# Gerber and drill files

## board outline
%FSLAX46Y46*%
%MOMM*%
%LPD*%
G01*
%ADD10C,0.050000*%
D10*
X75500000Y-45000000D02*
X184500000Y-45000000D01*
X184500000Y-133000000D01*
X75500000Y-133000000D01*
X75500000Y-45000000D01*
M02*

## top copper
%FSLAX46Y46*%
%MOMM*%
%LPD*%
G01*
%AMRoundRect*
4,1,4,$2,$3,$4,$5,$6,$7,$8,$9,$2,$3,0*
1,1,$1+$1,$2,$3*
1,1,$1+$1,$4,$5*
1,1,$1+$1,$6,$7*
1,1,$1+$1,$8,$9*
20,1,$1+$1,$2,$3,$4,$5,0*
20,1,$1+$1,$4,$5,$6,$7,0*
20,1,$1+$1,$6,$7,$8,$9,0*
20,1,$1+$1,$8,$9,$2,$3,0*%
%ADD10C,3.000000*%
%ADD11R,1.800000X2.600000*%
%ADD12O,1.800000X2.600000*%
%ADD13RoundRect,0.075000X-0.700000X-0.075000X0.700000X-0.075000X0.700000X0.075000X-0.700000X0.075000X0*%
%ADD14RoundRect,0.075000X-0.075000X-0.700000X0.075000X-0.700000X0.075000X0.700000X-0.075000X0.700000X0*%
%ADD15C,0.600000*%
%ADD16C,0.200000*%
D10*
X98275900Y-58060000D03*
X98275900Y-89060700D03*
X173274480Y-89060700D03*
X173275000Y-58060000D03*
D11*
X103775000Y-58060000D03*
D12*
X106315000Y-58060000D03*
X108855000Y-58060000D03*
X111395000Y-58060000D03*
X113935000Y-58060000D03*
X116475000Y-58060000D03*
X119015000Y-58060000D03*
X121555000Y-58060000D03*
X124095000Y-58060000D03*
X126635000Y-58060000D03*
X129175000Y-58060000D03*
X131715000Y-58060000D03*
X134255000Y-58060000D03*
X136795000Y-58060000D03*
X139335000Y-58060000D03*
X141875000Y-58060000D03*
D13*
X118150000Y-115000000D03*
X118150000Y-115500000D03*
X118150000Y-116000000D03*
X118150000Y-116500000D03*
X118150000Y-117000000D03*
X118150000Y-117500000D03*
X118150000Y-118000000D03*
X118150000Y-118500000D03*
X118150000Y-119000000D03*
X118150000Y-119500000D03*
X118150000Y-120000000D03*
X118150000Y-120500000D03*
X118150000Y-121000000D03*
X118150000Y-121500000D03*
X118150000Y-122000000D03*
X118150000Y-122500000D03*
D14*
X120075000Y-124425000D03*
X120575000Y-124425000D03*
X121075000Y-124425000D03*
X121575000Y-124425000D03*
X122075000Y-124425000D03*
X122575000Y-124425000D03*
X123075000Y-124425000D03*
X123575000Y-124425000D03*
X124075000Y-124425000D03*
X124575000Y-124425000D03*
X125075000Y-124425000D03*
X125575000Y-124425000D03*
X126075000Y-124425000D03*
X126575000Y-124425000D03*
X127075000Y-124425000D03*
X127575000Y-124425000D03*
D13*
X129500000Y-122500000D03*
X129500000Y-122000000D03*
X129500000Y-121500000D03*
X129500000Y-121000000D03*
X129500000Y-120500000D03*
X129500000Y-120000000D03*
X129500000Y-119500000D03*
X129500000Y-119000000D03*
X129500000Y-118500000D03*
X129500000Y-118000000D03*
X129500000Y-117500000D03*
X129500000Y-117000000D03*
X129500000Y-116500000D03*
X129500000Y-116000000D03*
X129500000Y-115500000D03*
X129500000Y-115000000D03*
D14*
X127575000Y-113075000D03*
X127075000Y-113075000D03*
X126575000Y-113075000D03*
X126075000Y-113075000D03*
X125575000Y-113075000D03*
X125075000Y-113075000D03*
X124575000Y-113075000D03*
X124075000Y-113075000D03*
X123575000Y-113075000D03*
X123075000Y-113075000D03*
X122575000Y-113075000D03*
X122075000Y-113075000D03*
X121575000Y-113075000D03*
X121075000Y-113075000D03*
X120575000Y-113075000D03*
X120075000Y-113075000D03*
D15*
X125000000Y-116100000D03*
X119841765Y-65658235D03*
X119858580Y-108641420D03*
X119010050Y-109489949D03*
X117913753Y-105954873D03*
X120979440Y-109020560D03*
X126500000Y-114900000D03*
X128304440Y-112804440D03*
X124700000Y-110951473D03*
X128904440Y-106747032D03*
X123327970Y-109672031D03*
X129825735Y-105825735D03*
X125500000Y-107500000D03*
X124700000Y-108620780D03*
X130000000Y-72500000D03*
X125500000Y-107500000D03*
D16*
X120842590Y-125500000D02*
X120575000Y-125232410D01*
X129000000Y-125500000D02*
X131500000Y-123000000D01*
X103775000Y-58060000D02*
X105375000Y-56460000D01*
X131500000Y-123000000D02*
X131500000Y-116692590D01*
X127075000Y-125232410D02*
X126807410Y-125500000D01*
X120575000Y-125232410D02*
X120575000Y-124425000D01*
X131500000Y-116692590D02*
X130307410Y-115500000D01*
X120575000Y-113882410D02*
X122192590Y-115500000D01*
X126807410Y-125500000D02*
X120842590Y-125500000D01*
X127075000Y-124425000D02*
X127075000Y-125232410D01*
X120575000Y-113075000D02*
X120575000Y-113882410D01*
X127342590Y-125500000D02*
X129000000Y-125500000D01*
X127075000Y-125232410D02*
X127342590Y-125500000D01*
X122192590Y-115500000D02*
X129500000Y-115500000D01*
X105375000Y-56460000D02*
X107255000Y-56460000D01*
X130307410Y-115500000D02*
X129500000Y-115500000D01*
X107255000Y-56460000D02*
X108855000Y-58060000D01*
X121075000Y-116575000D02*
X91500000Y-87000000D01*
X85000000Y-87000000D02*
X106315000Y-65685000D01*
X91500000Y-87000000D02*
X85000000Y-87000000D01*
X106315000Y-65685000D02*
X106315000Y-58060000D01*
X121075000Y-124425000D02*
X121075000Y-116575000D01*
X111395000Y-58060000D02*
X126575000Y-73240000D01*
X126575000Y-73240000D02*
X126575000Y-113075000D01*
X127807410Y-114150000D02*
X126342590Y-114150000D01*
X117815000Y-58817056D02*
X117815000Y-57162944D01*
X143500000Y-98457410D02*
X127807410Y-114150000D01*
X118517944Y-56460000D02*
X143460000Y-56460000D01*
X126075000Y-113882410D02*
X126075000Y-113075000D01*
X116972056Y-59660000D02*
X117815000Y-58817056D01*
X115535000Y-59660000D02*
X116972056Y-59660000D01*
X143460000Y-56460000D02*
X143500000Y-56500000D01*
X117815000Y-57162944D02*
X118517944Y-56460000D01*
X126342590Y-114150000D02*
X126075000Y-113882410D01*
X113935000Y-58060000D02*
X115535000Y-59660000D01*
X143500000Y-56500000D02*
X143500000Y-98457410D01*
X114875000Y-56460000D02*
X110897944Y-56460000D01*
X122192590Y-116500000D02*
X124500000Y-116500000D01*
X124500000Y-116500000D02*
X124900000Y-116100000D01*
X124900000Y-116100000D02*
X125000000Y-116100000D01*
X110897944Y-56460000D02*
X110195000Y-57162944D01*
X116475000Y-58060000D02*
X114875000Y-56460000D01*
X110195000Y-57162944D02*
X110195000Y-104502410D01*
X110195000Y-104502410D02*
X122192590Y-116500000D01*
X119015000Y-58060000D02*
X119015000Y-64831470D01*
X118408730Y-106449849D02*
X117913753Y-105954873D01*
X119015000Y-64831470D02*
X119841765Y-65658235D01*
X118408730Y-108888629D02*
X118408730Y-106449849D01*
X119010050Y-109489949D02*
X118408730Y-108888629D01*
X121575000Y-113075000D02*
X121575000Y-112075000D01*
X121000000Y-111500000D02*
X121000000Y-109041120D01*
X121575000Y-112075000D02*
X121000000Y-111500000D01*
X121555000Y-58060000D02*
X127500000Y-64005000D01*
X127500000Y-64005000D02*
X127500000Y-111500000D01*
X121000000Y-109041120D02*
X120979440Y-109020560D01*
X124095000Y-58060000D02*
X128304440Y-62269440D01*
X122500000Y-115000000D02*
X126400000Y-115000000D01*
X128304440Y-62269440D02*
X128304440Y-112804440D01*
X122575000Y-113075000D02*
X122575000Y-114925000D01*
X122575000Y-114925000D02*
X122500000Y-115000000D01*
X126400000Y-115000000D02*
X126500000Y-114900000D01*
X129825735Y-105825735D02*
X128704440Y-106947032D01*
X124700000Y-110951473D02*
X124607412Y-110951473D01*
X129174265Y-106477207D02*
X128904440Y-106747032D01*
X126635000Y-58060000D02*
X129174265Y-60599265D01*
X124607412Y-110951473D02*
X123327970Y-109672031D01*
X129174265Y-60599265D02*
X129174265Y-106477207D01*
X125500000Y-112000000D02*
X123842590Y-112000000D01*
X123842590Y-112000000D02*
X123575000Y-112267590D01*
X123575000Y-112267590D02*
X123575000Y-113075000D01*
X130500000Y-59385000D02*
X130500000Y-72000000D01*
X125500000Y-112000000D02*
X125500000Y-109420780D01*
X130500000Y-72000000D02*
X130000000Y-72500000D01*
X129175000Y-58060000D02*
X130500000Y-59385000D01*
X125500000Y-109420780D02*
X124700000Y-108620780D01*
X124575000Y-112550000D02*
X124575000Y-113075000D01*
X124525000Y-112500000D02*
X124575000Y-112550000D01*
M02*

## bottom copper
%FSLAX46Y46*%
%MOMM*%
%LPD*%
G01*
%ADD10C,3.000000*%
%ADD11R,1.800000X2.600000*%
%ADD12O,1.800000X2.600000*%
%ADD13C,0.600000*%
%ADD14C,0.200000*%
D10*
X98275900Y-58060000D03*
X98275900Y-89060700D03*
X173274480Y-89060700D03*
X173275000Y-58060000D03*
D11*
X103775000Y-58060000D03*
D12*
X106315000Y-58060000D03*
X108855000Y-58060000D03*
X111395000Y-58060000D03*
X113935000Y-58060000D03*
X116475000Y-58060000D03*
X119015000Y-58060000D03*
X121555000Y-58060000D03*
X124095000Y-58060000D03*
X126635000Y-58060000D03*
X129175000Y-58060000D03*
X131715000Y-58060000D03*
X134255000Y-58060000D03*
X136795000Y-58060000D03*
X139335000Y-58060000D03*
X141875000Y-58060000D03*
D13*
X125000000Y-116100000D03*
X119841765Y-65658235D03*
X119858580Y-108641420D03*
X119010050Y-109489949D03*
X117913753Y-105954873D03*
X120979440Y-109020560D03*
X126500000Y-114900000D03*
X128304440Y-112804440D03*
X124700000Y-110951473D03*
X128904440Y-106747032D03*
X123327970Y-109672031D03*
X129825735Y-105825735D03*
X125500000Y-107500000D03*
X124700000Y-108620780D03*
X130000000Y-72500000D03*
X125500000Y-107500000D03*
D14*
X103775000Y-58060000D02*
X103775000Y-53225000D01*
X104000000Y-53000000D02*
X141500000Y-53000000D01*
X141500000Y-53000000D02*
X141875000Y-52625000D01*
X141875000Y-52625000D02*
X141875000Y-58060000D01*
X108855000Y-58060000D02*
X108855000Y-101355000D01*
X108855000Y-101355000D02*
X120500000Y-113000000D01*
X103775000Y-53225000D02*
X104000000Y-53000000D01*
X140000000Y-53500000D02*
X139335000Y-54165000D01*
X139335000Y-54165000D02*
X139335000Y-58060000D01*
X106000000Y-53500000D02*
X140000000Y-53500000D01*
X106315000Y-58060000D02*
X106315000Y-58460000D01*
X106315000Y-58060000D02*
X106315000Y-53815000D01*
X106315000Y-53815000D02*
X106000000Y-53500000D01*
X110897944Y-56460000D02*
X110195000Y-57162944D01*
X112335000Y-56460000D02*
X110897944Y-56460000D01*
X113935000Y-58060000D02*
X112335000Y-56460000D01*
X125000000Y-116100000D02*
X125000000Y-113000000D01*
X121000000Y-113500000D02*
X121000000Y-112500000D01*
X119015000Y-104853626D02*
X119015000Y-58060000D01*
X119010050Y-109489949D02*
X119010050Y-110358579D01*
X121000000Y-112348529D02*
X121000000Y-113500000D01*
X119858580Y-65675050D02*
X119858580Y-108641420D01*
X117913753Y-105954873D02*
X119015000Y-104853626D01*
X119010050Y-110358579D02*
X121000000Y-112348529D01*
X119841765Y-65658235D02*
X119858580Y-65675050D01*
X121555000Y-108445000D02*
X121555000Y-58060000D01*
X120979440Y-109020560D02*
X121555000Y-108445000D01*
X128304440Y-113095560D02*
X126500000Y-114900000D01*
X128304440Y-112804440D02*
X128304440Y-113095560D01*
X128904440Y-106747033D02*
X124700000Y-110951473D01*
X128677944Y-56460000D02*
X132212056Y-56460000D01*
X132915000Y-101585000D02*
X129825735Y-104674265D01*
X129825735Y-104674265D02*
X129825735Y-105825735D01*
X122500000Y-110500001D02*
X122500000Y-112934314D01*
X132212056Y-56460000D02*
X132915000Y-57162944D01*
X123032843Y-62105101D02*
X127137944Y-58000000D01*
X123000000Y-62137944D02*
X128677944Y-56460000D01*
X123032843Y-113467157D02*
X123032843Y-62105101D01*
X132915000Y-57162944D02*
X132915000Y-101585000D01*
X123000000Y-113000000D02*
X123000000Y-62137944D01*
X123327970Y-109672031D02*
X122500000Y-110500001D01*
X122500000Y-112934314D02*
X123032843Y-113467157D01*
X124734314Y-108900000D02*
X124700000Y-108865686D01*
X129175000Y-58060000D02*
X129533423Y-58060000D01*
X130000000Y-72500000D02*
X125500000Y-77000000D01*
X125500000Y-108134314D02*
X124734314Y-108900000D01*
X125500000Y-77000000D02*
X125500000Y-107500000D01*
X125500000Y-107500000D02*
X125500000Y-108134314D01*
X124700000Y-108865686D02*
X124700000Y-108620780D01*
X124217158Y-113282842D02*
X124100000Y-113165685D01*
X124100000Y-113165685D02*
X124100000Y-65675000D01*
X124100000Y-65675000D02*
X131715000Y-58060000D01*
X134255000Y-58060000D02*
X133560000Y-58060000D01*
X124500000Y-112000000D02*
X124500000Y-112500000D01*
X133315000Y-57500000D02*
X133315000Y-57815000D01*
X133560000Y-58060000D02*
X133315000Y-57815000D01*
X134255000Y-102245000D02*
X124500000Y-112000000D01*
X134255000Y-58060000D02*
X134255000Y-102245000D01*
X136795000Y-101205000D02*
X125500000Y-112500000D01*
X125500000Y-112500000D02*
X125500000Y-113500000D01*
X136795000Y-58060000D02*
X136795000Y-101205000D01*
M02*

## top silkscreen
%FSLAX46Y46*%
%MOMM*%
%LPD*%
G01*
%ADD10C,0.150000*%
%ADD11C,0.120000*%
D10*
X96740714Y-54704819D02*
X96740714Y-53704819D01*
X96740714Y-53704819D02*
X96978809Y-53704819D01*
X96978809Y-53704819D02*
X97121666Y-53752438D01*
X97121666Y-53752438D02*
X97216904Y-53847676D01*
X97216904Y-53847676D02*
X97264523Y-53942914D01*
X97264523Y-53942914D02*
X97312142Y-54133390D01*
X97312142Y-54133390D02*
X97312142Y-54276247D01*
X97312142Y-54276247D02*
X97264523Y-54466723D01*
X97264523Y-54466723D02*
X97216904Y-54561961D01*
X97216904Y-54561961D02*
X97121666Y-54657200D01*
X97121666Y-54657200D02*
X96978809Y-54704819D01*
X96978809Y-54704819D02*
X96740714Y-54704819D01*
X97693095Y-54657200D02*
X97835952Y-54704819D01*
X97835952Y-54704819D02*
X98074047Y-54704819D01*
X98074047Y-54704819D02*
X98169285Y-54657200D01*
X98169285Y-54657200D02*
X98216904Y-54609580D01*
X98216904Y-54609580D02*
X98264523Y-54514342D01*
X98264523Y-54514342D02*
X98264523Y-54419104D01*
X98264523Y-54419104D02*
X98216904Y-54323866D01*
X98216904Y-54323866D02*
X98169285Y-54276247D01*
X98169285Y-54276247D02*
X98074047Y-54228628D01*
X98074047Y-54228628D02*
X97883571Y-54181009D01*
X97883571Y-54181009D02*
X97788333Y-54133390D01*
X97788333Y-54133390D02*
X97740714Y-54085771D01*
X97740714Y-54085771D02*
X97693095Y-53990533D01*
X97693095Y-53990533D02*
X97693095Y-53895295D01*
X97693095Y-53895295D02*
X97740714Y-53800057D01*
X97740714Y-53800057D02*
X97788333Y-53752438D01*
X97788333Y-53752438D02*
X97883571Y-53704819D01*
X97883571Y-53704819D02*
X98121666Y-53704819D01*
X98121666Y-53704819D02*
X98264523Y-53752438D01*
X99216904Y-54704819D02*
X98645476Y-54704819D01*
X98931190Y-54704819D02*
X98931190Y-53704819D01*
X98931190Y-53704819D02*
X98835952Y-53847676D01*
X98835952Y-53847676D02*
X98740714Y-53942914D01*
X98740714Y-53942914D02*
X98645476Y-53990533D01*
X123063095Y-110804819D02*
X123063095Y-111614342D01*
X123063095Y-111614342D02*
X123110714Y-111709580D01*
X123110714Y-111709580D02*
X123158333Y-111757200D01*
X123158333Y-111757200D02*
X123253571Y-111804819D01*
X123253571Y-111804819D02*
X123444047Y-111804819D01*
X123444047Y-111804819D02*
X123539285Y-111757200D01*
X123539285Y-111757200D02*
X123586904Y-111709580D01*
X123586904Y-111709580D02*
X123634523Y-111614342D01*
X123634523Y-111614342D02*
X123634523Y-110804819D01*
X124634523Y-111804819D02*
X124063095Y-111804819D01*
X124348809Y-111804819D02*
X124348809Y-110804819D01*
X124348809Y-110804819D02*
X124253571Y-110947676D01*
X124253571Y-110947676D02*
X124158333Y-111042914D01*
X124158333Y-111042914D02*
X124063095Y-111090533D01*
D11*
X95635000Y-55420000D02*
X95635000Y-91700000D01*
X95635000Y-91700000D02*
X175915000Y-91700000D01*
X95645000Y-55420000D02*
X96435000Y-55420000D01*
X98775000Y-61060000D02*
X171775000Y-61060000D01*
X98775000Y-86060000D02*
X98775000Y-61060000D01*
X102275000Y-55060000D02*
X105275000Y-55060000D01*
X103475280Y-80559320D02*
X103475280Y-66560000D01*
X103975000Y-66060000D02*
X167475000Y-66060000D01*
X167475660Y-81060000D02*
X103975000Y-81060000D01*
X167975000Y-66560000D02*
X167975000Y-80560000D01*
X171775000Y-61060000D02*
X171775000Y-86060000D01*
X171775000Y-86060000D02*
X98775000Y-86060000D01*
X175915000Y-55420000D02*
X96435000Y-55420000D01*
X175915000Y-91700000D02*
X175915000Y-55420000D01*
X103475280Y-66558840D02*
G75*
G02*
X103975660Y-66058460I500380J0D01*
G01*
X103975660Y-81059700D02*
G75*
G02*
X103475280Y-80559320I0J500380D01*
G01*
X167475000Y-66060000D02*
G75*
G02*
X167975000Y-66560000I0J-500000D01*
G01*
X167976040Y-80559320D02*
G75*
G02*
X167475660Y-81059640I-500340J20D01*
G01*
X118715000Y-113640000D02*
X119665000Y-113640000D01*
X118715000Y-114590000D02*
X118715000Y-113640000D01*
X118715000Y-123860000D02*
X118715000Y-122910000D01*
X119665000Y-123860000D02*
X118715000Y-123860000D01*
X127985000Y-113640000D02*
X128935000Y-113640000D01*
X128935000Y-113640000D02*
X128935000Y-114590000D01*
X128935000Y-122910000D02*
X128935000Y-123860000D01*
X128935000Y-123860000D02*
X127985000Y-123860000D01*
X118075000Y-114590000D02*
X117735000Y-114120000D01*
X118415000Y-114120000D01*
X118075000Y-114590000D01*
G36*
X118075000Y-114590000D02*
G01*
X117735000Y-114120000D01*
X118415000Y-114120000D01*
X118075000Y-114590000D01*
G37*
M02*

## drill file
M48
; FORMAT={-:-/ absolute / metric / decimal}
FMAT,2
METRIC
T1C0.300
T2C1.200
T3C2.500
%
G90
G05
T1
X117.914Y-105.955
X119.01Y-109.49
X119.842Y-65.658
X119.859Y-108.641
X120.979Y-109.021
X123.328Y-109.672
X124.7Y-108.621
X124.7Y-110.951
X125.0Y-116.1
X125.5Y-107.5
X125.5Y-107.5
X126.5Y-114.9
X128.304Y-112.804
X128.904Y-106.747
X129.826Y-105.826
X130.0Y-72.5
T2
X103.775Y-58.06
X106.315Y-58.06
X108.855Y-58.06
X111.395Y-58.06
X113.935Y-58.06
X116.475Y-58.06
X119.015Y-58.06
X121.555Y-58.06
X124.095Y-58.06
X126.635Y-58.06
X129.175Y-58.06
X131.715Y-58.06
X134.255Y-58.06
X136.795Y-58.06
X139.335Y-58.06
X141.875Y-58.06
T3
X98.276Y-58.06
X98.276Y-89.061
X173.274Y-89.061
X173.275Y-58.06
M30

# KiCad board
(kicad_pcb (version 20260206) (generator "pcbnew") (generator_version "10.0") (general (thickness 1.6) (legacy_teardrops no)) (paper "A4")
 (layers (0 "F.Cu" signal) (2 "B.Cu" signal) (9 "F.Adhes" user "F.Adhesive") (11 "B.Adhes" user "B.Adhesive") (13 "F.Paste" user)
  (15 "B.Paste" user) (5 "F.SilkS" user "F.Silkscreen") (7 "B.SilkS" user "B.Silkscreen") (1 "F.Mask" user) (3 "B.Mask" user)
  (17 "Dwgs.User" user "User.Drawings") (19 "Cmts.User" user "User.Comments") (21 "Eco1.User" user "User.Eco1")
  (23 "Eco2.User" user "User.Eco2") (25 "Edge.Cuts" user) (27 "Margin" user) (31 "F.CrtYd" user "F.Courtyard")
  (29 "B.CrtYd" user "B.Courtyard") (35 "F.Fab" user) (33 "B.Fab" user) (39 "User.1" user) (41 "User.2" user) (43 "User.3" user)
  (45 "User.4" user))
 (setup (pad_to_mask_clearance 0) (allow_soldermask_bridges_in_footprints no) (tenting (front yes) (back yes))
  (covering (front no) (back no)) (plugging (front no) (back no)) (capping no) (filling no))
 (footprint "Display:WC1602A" (layer "F.Cu") (at 103.775 58.06)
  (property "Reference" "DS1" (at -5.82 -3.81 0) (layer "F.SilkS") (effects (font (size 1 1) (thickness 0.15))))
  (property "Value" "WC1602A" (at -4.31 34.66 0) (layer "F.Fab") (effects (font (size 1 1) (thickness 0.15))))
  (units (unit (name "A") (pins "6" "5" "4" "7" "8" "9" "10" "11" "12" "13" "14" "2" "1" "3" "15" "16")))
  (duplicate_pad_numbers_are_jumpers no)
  (fp_line (start -8.14 -2.64) (end -8.14 33.64) (stroke (width 0.12) (type solid)) (layer "F.SilkS"))
  (fp_line (start -8.14 33.64) (end 72.14 33.64) (stroke (width 0.12) (type solid)) (layer "F.SilkS"))
  (fp_line (start -8.13 -2.64) (end -7.34 -2.64) (stroke (width 0.12) (type solid)) (layer "F.SilkS"))
  (fp_line (start -5 3) (end 68 3) (stroke (width 0.12) (type solid)) (layer "F.SilkS"))
  (fp_line (start -5 28) (end -5 3) (stroke (width 0.12) (type solid)) (layer "F.SilkS"))
  (fp_line (start -1.5 -3) (end 1.5 -3) (stroke (width 0.12) (type solid)) (layer "F.SilkS"))
  (fp_line (start -0.29972 22.49932) (end -0.29972 8.5) (stroke (width 0.12) (type solid)) (layer "F.SilkS"))
  (fp_line (start 0.2 8) (end 63.7 8) (stroke (width 0.12) (type solid)) (layer "F.SilkS"))
  (fp_line (start 63.70066 23) (end 0.2 23) (stroke (width 0.12) (type solid)) (layer "F.SilkS"))
  (fp_line (start 64.2 8.5) (end 64.2 22.5) (stroke (width 0.12) (type solid)) (layer "F.SilkS"))
  (fp_line (start 68 3) (end 68 28) (stroke (width 0.12) (type solid)) (layer "F.SilkS"))
  (fp_line (start 68 28) (end -5 28) (stroke (width 0.12) (type solid)) (layer "F.SilkS"))
  (fp_line (start 72.14 -2.64) (end -7.34 -2.64) (stroke (width 0.12) (type solid)) (layer "F.SilkS"))
  (fp_line (start 72.14 33.64) (end 72.14 -2.64) (stroke (width 0.12) (type solid)) (layer "F.SilkS"))
  (fp_arc (start -0.29972 8.49884) (mid -0.153162 8.145018) (end 0.20066 7.99846) (stroke (width 0.12) (type solid)) (layer "F.SilkS"))
  (fp_arc (start 0.20066 22.9997) (mid -0.153162 22.853142) (end -0.29972 22.49932) (stroke (width 0.12) (type solid)) (layer "F.SilkS"))
  (fp_arc (start 63.7 8) (mid 64.053553 8.146447) (end 64.2 8.5) (stroke (width 0.12) (type solid)) (layer "F.SilkS"))
  (fp_arc (start 64.20104 22.49932) (mid 64.054482 22.853142) (end 63.70066 22.9997) (stroke (width 0.12) (type solid)) (layer "F.SilkS"))
  (pad "" thru_hole circle (at -5.4991 0) (size 3 3) (drill 2.5) (layers "*.Cu" "*.Mask") (remove_unused_layers no))
  (pad "" thru_hole circle (at -5.4991 31.0007) (size 3 3) (drill 2.5) (layers "*.Cu" "*.Mask") (remove_unused_layers no))
  (pad "" thru_hole circle (at 69.49948 31.0007) (size 3 3) (drill 2.5) (layers "*.Cu" "*.Mask") (remove_unused_layers no))
  (pad "" thru_hole circle (at 69.5 0) (size 3 3) (drill 2.5) (layers "*.Cu" "*.Mask") (remove_unused_layers no))
  (pad "1" thru_hole rect (at 0 0) (size 1.8 2.6) (drill 1.2) (layers "*.Cu" "*.Mask") (remove_unused_layers no) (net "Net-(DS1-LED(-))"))
  (pad "2" thru_hole oval (at 2.54 0) (size 1.8 2.6) (drill 1.2) (layers "*.Cu" "*.Mask") (remove_unused_layers no) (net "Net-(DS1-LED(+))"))
  (pad "3" thru_hole oval (at 5.08 0) (size 1.8 2.6) (drill 1.2) (layers "*.Cu" "*.Mask") (remove_unused_layers no) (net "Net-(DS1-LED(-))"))
  (pad "4" thru_hole oval (at 7.62 0) (size 1.8 2.6) (drill 1.2) (layers "*.Cu" "*.Mask") (remove_unused_layers no) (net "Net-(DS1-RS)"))
  (pad "5" thru_hole oval (at 10.16 0) (size 1.8 2.6) (drill 1.2) (layers "*.Cu" "*.Mask") (remove_unused_layers no)
   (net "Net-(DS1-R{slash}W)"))
  (pad "6" thru_hole oval (at 12.7 0) (size 1.8 2.6) (drill 1.2) (layers "*.Cu" "*.Mask") (remove_unused_layers no) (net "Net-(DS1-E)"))
  (pad "7" thru_hole oval (at 15.24 0) (size 1.8 2.6) (drill 1.2) (layers "*.Cu" "*.Mask") (remove_unused_layers no) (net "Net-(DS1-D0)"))
  (pad "8" thru_hole oval (at 17.78 0) (size 1.8 2.6) (drill 1.2) (layers "*.Cu" "*.Mask") (remove_unused_layers no) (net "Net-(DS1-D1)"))
  (pad "9" thru_hole oval (at 20.32 0) (size 1.8 2.6) (drill 1.2) (layers "*.Cu" "*.Mask") (remove_unused_layers no) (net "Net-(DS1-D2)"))
  (pad "10" thru_hole oval (at 22.86 0) (size 1.8 2.6) (drill 1.2) (layers "*.Cu" "*.Mask") (remove_unused_layers no) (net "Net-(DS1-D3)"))
  (pad "11" thru_hole oval (at 25.4 0) (size 1.8 2.6) (drill 1.2) (layers "*.Cu" "*.Mask") (remove_unused_layers no) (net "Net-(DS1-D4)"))
  (pad "12" thru_hole oval (at 27.94 0) (size 1.8 2.6) (drill 1.2) (layers "*.Cu" "*.Mask") (remove_unused_layers no) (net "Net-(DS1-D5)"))
  (pad "13" thru_hole oval (at 30.48 0) (size 1.8 2.6) (drill 1.2) (layers "*.Cu" "*.Mask") (remove_unused_layers no) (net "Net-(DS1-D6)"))
  (pad "14" thru_hole oval (at 33.02 0) (size 1.8 2.6) (drill 1.2) (layers "*.Cu" "*.Mask") (remove_unused_layers no) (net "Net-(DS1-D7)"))
  (pad "15" thru_hole oval (at 35.56 0) (size 1.8 2.6) (drill 1.2) (layers "*.Cu" "*.Mask") (remove_unused_layers no)
   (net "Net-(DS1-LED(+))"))
  (pad "16" thru_hole oval (at 38.1 0) (size 1.8 2.6) (drill 1.2) (layers "*.Cu" "*.Mask") (remove_unused_layers no)
   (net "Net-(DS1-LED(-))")))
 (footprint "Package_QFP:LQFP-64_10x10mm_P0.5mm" (layer "F.Cu") (at 123.825 118.75)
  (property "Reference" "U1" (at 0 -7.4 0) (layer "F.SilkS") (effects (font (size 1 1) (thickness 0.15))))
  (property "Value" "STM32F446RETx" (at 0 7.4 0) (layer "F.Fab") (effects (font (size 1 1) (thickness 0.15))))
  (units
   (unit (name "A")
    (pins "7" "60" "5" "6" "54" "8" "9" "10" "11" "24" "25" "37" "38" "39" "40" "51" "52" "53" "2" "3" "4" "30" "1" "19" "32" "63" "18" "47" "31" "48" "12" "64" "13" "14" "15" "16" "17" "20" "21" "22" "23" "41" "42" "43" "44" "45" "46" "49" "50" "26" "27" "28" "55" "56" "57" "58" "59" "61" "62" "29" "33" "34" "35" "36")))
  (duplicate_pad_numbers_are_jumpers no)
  (fp_line (start -5.11 -5.11) (end -4.16 -5.11) (stroke (width 0.12) (type solid)) (layer "F.SilkS"))
  (fp_line (start -5.11 -4.16) (end -5.11 -5.11) (stroke (width 0.12) (type solid)) (layer "F.SilkS"))
  (fp_line (start -5.11 5.11) (end -5.11 4.16) (stroke (width 0.12) (type solid)) (layer "F.SilkS"))
  (fp_line (start -4.16 5.11) (end -5.11 5.11) (stroke (width 0.12) (type solid)) (layer "F.SilkS"))
  (fp_line (start 4.16 -5.11) (end 5.11 -5.11) (stroke (width 0.12) (type solid)) (layer "F.SilkS"))
  (fp_line (start 5.11 -5.11) (end 5.11 -4.16) (stroke (width 0.12) (type solid)) (layer "F.SilkS"))
  (fp_line (start 5.11 4.16) (end 5.11 5.11) (stroke (width 0.12) (type solid)) (layer "F.SilkS"))
  (fp_line (start 5.11 5.11) (end 4.16 5.11) (stroke (width 0.12) (type solid)) (layer "F.SilkS"))
  (fp_poly (pts (xy -5.75 -4.16) (xy -6.09 -4.63) (xy -5.41 -4.63)) (stroke (width 0.12) (type solid)) (fill yes) (layer "F.SilkS"))
  (pad "1" smd roundrect (at -5.675 -3.75) (size 1.55 0.3) (layers "F.Cu" "F.Mask" "F.Paste") (roundrect_rratio 0.25)
   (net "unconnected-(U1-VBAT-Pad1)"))
  (pad "2" smd roundrect (at -5.675 -3.25) (size 1.55 0.3) (layers "F.Cu" "F.Mask" "F.Paste") (roundrect_rratio 0.25)
   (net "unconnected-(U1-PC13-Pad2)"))
  (pad "3" smd roundrect (at -5.675 -2.75) (size 1.55 0.3) (layers "F.Cu" "F.Mask" "F.Paste") (roundrect_rratio 0.25)
   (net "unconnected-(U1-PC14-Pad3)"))
  (pad "4" smd roundrect (at -5.675 -2.25) (size 1.55 0.3) (layers "F.Cu" "F.Mask" "F.Paste") (roundrect_rratio 0.25)
   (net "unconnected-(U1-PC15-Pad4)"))
  (pad "5" smd roundrect (at -5.675 -1.75) (size 1.55 0.3) (layers "F.Cu" "F.Mask" "F.Paste") (roundrect_rratio 0.25)
   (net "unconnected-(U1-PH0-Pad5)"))
  (pad "6" smd roundrect (at -5.675 -1.25) (size 1.55 0.3) (layers "F.Cu" "F.Mask" "F.Paste") (roundrect_rratio 0.25)
   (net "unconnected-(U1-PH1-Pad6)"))
  (pad "7" smd roundrect (at -5.675 -0.75) (size 1.55 0.3) (layers "F.Cu" "F.Mask" "F.Paste") (roundrect_rratio 0.25)
   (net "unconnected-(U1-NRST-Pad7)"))
  (pad "8" smd roundrect (at -5.675 -0.25) (size 1.55 0.3) (layers "F.Cu" "F.Mask" "F.Paste") (roundrect_rratio 0.25)
   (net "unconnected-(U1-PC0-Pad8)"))
  (pad "9" smd roundrect (at -5.675 0.25) (size 1.55 0.3) (layers "F.Cu" "F.Mask" "F.Paste") (roundrect_rratio 0.25)
   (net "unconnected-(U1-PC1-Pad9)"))
  (pad "10" smd roundrect (at -5.675 0.75) (size 1.55 0.3) (layers "F.Cu" "F.Mask" "F.Paste") (roundrect_rratio 0.25)
   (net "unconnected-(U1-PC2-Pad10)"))
  (pad "11" smd roundrect (at -5.675 1.25) (size 1.55 0.3) (layers "F.Cu" "F.Mask" "F.Paste") (roundrect_rratio 0.25)
   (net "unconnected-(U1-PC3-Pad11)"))
  (pad "12" smd roundrect (at -5.675 1.75) (size 1.55 0.3) (layers "F.Cu" "F.Mask" "F.Paste") (roundrect_rratio 0.25)
   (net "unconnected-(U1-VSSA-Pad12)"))
  (pad "13" smd roundrect (at -5.675 2.25) (size 1.55 0.3) (layers "F.Cu" "F.Mask" "F.Paste") (roundrect_rratio 0.25)
   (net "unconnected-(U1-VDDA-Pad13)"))
  (pad "14" smd roundrect (at -5.675 2.75) (size 1.55 0.3) (layers "F.Cu" "F.Mask" "F.Paste") (roundrect_rratio 0.25)
   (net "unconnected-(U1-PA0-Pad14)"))
  (pad "15" smd roundrect (at -5.675 3.25) (size 1.55 0.3) (layers "F.Cu" "F.Mask" "F.Paste") (roundrect_rratio 0.25)
   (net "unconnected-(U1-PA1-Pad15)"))
  (pad "16" smd roundrect (at -5.675 3.75) (size 1.55 0.3) (layers "F.Cu" "F.Mask" "F.Paste") (roundrect_rratio 0.25)
   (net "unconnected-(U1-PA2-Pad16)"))
  (pad "17" smd roundrect (at -3.75 5.675) (size 0.3 1.55) (layers "F.Cu" "F.Mask" "F.Paste") (roundrect_rratio 0.25)
   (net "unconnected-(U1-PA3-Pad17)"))
  (pad "18" smd roundrect (at -3.25 5.675) (size 0.3 1.55) (layers "F.Cu" "F.Mask" "F.Paste") (roundrect_rratio 0.25)
   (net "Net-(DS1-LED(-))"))
  (pad "19" smd roundrect (at -2.75 5.675) (size 0.3 1.55) (layers "F.Cu" "F.Mask" "F.Paste") (roundrect_rratio 0.25)
   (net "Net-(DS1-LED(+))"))
  (pad "20" smd roundrect (at -2.25 5.675) (size 0.3 1.55) (layers "F.Cu" "F.Mask" "F.Paste") (roundrect_rratio 0.25)
   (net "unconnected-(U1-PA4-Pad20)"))
  (pad "21" smd roundrect (at -1.75 5.675) (size 0.3 1.55) (layers "F.Cu" "F.Mask" "F.Paste") (roundrect_rratio 0.25)
   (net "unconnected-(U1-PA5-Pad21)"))
  (pad "22" smd roundrect (at -1.25 5.675) (size 0.3 1.55) (layers "F.Cu" "F.Mask" "F.Paste") (roundrect_rratio 0.25)
   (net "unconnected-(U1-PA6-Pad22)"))
  (pad "23" smd roundrect (at -0.75 5.675) (size 0.3 1.55) (layers "F.Cu" "F.Mask" "F.Paste") (roundrect_rratio 0.25)
   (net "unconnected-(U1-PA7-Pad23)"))
  (pad "24" smd roundrect (at -0.25 5.675) (size 0.3 1.55) (layers "F.Cu" "F.Mask" "F.Paste") (roundrect_rratio 0.25)
   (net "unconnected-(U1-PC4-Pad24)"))
  (pad "25" smd roundrect (at 0.25 5.675) (size 0.3 1.55) (layers "F.Cu" "F.Mask" "F.Paste") (roundrect_rratio 0.25)
   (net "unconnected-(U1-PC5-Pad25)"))
  (pad "26" smd roundrect (at 0.75 5.675) (size 0.3 1.55) (layers "F.Cu" "F.Mask" "F.Paste") (roundrect_rratio 0.25)
   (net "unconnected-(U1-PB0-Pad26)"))
  (pad "27" smd roundrect (at 1.25 5.675) (size 0.3 1.55) (layers "F.Cu" "F.Mask" "F.Paste") (roundrect_rratio 0.25)
   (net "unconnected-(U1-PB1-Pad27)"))
  (pad "28" smd roundrect (at 1.75 5.675) (size 0.3 1.55) (layers "F.Cu" "F.Mask" "F.Paste") (roundrect_rratio 0.25)
   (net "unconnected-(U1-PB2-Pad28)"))
  (pad "29" smd roundrect (at 2.25 5.675) (size 0.3 1.55) (layers "F.Cu" "F.Mask" "F.Paste") (roundrect_rratio 0.25)
   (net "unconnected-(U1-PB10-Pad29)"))
  (pad "30" smd roundrect (at 2.75 5.675) (size 0.3 1.55) (layers "F.Cu" "F.Mask" "F.Paste") (roundrect_rratio 0.25)
   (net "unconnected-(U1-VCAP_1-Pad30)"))
  (pad "31" smd roundrect (at 3.25 5.675) (size 0.3 1.55) (layers "F.Cu" "F.Mask" "F.Paste") (roundrect_rratio 0.25)
   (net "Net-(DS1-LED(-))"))
  (pad "32" smd roundrect (at 3.75 5.675) (size 0.3 1.55) (layers "F.Cu" "F.Mask" "F.Paste") (roundrect_rratio 0.25)
   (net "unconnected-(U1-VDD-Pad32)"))
  (pad "33" smd roundrect (at 5.675 3.75) (size 1.55 0.3) (layers "F.Cu" "F.Mask" "F.Paste") (roundrect_rratio 0.25)
   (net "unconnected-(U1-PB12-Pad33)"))
  (pad "34" smd roundrect (at 5.675 3.25) (size 1.55 0.3) (layers "F.Cu" "F.Mask" "F.Paste") (roundrect_rratio 0.25)
   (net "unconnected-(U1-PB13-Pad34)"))
  (pad "35" smd roundrect (at 5.675 2.75) (size 1.55 0.3) (layers "F.Cu" "F.Mask" "F.Paste") (roundrect_rratio 0.25)
   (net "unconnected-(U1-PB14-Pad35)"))
  (pad "36" smd roundrect (at 5.675 2.25) (size 1.55 0.3) (layers "F.Cu" "F.Mask" "F.Paste") (roundrect_rratio 0.25)
   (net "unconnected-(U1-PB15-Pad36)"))
  (pad "37" smd roundrect (at 5.675 1.75) (size 1.55 0.3) (layers "F.Cu" "F.Mask" "F.Paste") (roundrect_rratio 0.25)
   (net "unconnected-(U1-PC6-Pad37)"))
  (pad "38" smd roundrect (at 5.675 1.25) (size 1.55 0.3) (layers "F.Cu" "F.Mask" "F.Paste") (roundrect_rratio 0.25)
   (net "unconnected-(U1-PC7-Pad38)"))
  (pad "39" smd roundrect (at 5.675 0.75) (size 1.55 0.3) (layers "F.Cu" "F.Mask" "F.Paste") (roundrect_rratio 0.25)
   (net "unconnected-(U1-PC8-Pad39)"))
  (pad "40" smd roundrect (at 5.675 0.25) (size 1.55 0.3) (layers "F.Cu" "F.Mask" "F.Paste") (roundrect_rratio 0.25)
   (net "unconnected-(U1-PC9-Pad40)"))
  (pad "41" smd roundrect (at 5.675 -0.25) (size 1.55 0.3) (layers "F.Cu" "F.Mask" "F.Paste") (roundrect_rratio 0.25)
   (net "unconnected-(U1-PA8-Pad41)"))
  (pad "42" smd roundrect (at 5.675 -0.75) (size 1.55 0.3) (layers "F.Cu" "F.Mask" "F.Paste") (roundrect_rratio 0.25)
   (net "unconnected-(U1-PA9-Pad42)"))
  (pad "43" smd roundrect (at 5.675 -1.25) (size 1.55 0.3) (layers "F.Cu" "F.Mask" "F.Paste") (roundrect_rratio 0.25)
   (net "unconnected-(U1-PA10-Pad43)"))
  (pad "44" smd roundrect (at 5.675 -1.75) (size 1.55 0.3) (layers "F.Cu" "F.Mask" "F.Paste") (roundrect_rratio 0.25)
   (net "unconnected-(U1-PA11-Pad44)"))
  (pad "45" smd roundrect (at 5.675 -2.25) (size 1.55 0.3) (layers "F.Cu" "F.Mask" "F.Paste") (roundrect_rratio 0.25)
   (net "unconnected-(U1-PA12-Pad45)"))
  (pad "46" smd roundrect (at 5.675 -2.75) (size 1.55 0.3) (layers "F.Cu" "F.Mask" "F.Paste") (roundrect_rratio 0.25)
   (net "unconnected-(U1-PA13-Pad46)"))
  (pad "47" smd roundrect (at 5.675 -3.25) (size 1.55 0.3) (layers "F.Cu" "F.Mask" "F.Paste") (roundrect_rratio 0.25)
   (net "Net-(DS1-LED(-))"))
  (pad "48" smd roundrect (at 5.675 -3.75) (size 1.55 0.3) (layers "F.Cu" "F.Mask" "F.Paste") (roundrect_rratio 0.25)
   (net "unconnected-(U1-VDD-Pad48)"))
  (pad "49" smd roundrect (at 3.75 -5.675) (size 0.3 1.55) (layers "F.Cu" "F.Mask" "F.Paste") (roundrect_rratio 0.25)
   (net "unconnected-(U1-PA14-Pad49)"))
  (pad "50" smd roundrect (at 3.25 -5.675) (size 0.3 1.55) (layers "F.Cu" "F.Mask" "F.Paste") (roundrect_rratio 0.25)
   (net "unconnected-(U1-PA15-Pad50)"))
  (pad "51" smd roundrect (at 2.75 -5.675) (size 0.3 1.55) (layers "F.Cu" "F.Mask" "F.Paste") (roundrect_rratio 0.25) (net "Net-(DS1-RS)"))
  (pad "52" smd roundrect (at 2.25 -5.675) (size 0.3 1.55) (layers "F.Cu" "F.Mask" "F.Paste") (roundrect_rratio 0.25)
   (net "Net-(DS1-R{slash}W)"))
  (pad "53" smd roundrect (at 1.75 -5.675) (size 0.3 1.55) (layers "F.Cu" "F.Mask" "F.Paste") (roundrect_rratio 0.25) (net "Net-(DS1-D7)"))
  (pad "54" smd roundrect (at 1.25 -5.675) (size 0.3 1.55) (layers "F.Cu" "F.Mask" "F.Paste") (roundrect_rratio 0.25) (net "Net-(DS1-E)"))
  (pad "55" smd roundrect (at 0.75 -5.675) (size 0.3 1.55) (layers "F.Cu" "F.Mask" "F.Paste") (roundrect_rratio 0.25) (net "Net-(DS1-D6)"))
  (pad "56" smd roundrect (at 0.25 -5.675) (size 0.3 1.55) (layers "F.Cu" "F.Mask" "F.Paste") (roundrect_rratio 0.25) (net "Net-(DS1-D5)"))
  (pad "57" smd roundrect (at -0.25 -5.675) (size 0.3 1.55) (layers "F.Cu" "F.Mask" "F.Paste") (roundrect_rratio 0.25) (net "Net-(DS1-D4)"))
  (pad "58" smd roundrect (at -0.75 -5.675) (size 0.3 1.55) (layers "F.Cu" "F.Mask" "F.Paste") (roundrect_rratio 0.25) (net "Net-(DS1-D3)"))
  (pad "59" smd roundrect (at -1.25 -5.675) (size 0.3 1.55) (layers "F.Cu" "F.Mask" "F.Paste") (roundrect_rratio 0.25) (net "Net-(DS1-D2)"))
  (pad "60" smd roundrect (at -1.75 -5.675) (size 0.3 1.55) (layers "F.Cu" "F.Mask" "F.Paste") (roundrect_rratio 0.25)
   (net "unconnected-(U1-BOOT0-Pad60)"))
  (pad "61" smd roundrect (at -2.25 -5.675) (size 0.3 1.55) (layers "F.Cu" "F.Mask" "F.Paste") (roundrect_rratio 0.25) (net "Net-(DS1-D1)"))
  (pad "62" smd roundrect (at -2.75 -5.675) (size 0.3 1.55) (layers "F.Cu" "F.Mask" "F.Paste") (roundrect_rratio 0.25) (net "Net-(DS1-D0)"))
  (pad "63" smd roundrect (at -3.25 -5.675) (size 0.3 1.55) (layers "F.Cu" "F.Mask" "F.Paste") (roundrect_rratio 0.25)
   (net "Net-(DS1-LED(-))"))
  (pad "64" smd roundrect (at -3.75 -5.675) (size 0.3 1.55) (layers "F.Cu" "F.Mask" "F.Paste") (roundrect_rratio 0.25)
   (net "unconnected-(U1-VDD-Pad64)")))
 (gr_rect (start 75.5 45) (end 184.5 133) (stroke (width 0.05) (type default)) (fill no) (layer "Edge.Cuts"))
 (segment (start 120.84259 125.5) (end 120.575 125.23241) (width 0.2) (layer "F.Cu") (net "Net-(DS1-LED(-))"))
 (segment (start 129 125.5) (end 131.5 123) (width 0.2) (layer "F.Cu") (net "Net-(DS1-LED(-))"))
 (segment (start 103.775 58.06) (end 105.375 56.46) (width 0.2) (layer "F.Cu") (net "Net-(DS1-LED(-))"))
 (segment (start 131.5 123) (end 131.5 116.69259) (width 0.2) (layer "F.Cu") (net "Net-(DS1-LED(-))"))
 (segment (start 127.075 125.23241) (end 126.80741 125.5) (width 0.2) (layer "F.Cu") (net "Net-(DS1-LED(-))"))
 (segment (start 120.575 125.23241) (end 120.575 124.425) (width 0.2) (layer "F.Cu") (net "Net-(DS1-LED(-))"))
 (segment (start 131.5 116.69259) (end 130.30741 115.5) (width 0.2) (layer "F.Cu") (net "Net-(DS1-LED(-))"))
 (segment (start 120.575 113.88241) (end 122.19259 115.5) (width 0.2) (layer "F.Cu") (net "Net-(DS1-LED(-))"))
 (segment (start 126.80741 125.5) (end 120.84259 125.5) (width 0.2) (layer "F.Cu") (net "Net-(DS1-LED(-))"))
 (segment (start 127.075 124.425) (end 127.075 125.23241) (width 0.2) (layer "F.Cu") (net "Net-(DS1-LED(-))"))
 (segment (start 120.575 113.075) (end 120.575 113.88241) (width 0.2) (layer "F.Cu") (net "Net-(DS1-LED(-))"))
 (segment (start 127.34259 125.5) (end 129 125.5) (width 0.2) (layer "F.Cu") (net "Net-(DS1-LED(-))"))
 (segment (start 127.075 125.23241) (end 127.34259 125.5) (width 0.2) (layer "F.Cu") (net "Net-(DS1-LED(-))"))
 (segment (start 122.19259 115.5) (end 129.5 115.5) (width 0.2) (layer "F.Cu") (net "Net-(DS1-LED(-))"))
 (segment (start 105.375 56.46) (end 107.255 56.46) (width 0.2) (layer "F.Cu") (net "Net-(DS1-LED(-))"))
 (segment (start 130.30741 115.5) (end 129.5 115.5) (width 0.2) (layer "F.Cu") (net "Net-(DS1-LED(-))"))
 (segment (start 107.255 56.46) (end 108.855 58.06) (width 0.2) (layer "F.Cu") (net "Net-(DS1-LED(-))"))
 (segment (start 103.775 58.06) (end 103.775 53.225) (width 0.2) (layer "B.Cu") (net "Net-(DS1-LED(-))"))
 (segment (start 104 53) (end 141.5 53) (width 0.2) (layer "B.Cu") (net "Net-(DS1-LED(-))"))
 (segment (start 141.5 53) (end 141.875 52.625) (width 0.2) (layer "B.Cu") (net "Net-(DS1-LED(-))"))
 (segment (start 141.875 52.625) (end 141.875 58.06) (width 0.2) (layer "B.Cu") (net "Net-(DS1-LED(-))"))
 (segment (start 108.855 58.06) (end 108.855 101.355) (width 0.2) (layer "B.Cu") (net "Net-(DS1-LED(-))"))
 (segment (start 108.855 101.355) (end 120.5 113) (width 0.2) (layer "B.Cu") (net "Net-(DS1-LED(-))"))
 (segment (start 103.775 53.225) (end 104 53) (width 0.2) (layer "B.Cu") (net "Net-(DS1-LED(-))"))
 (segment (start 121.075 116.575) (end 91.5 87) (width 0.2) (layer "F.Cu") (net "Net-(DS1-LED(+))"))
 (segment (start 85 87) (end 106.315 65.685) (width 0.2) (layer "F.Cu") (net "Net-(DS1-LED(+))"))
 (segment (start 91.5 87) (end 85 87) (width 0.2) (layer "F.Cu") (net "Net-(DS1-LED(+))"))
 (segment (start 106.315 65.685) (end 106.315 58.06) (width 0.2) (layer "F.Cu") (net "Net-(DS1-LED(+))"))
 (segment (start 121.075 124.425) (end 121.075 116.575) (width 0.2) (layer "F.Cu") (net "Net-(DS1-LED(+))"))
 (segment (start 140 53.5) (end 139.335 54.165) (width 0.2) (layer "B.Cu") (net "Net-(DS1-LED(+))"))
 (segment (start 139.335 54.165) (end 139.335 58.06) (width 0.2) (layer "B.Cu") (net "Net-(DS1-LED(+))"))
 (segment (start 106 53.5) (end 140 53.5) (width 0.2) (layer "B.Cu") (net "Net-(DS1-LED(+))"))
 (segment (start 106.315 58.06) (end 106.315 58.46) (width 0.2) (layer "B.Cu") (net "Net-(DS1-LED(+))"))
 (segment (start 106.315 58.06) (end 106.315 53.815) (width 0.2) (layer "B.Cu") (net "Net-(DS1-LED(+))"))
 (segment (start 106.315 53.815) (end 106 53.5) (width 0.2) (layer "B.Cu") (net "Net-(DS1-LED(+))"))
 (segment (start 111.395 58.06) (end 126.575 73.24) (width 0.2) (layer "F.Cu") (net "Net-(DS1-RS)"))
 (segment (start 126.575 73.24) (end 126.575 113.075) (width 0.2) (layer "F.Cu") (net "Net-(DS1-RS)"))
 (segment (start 127.80741 114.15) (end 126.34259 114.15) (width 0.2) (layer "F.Cu") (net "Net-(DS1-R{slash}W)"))
 (segment (start 117.815 58.817056) (end 117.815 57.162944) (width 0.2) (layer "F.Cu") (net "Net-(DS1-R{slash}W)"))
 (segment (start 143.5 98.45741) (end 127.80741 114.15) (width 0.2) (layer "F.Cu") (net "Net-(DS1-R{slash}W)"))
 (segment (start 118.517944 56.46) (end 143.46 56.46) (width 0.2) (layer "F.Cu") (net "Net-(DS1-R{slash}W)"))
 (segment (start 126.075 113.88241) (end 126.075 113.075) (width 0.2) (layer "F.Cu") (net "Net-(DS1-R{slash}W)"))
 (segment (start 116.972056 59.66) (end 117.815 58.817056) (width 0.2) (layer "F.Cu") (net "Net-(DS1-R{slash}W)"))
 (segment (start 115.535 59.66) (end 116.972056 59.66) (width 0.2) (layer "F.Cu") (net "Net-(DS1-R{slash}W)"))
 (segment (start 143.46 56.46) (end 143.5 56.5) (width 0.2) (layer "F.Cu") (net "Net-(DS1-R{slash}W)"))
 (segment (start 117.815 57.162944) (end 118.517944 56.46) (width 0.2) (layer "F.Cu") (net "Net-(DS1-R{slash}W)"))
 (segment (start 126.34259 114.15) (end 126.075 113.88241) (width 0.2) (layer "F.Cu") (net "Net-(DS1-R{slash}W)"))
 (segment (start 113.935 58.06) (end 115.535 59.66) (width 0.2) (layer "F.Cu") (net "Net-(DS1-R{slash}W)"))
 (segment (start 143.5 56.5) (end 143.5 98.45741) (width 0.2) (layer "F.Cu") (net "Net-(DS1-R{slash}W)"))
 (segment (start 110.897944 56.46) (end 110.195 57.162944) (width 0.2) (layer "B.Cu") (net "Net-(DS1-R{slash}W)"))
 (segment (start 112.335 56.46) (end 110.897944 56.46) (width 0.2) (layer "B.Cu") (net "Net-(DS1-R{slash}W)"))
 (segment (start 113.935 58.06) (end 112.335 56.46) (width 0.2) (layer "B.Cu") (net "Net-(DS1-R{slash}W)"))
 (segment (start 114.875 56.46) (end 110.897944 56.46) (width 0.2) (layer "F.Cu") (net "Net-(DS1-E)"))
 (segment (start 122.19259 116.5) (end 124.5 116.5) (width 0.2) (layer "F.Cu") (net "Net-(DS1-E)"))
 (segment (start 124.5 116.5) (end 124.9 116.1) (width 0.2) (layer "F.Cu") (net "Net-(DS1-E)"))
 (segment (start 124.9 116.1) (end 125 116.1) (width 0.2) (layer "F.Cu") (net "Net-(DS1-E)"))
 (segment (start 110.897944 56.46) (end 110.195 57.162944) (width 0.2) (layer "F.Cu") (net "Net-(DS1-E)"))
 (segment (start 116.475 58.06) (end 114.875 56.46) (width 0.2) (layer "F.Cu") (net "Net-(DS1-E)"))
 (segment (start 110.195 57.162944) (end 110.195 104.50241) (width 0.2) (layer "F.Cu") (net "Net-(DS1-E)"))
 (segment (start 110.195 104.50241) (end 122.19259 116.5) (width 0.2) (layer "F.Cu") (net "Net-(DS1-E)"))
 (via (at 125 116.1) (size 0.6) (drill 0.3) (layers "F.Cu" "B.Cu") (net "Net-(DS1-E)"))
 (segment (start 125 116.1) (end 125 113) (width 0.2) (layer "B.Cu") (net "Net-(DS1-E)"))
 (segment (start 119.015 58.06) (end 119.015 64.83147) (width 0.2) (layer "F.Cu") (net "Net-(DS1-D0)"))
 (segment (start 118.40873 106.449849) (end 117.913753 105.954873) (width 0.2) (layer "F.Cu") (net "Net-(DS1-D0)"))
 (segment (start 119.015 64.83147) (end 119.841765 65.658235) (width 0.2) (layer "F.Cu") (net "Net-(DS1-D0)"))
 (segment (start 118.40873 108.888629) (end 118.40873 106.449849) (width 0.2) (layer "F.Cu") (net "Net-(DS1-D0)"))
 (segment (start 119.01005 109.489949) (end 118.40873 108.888629) (width 0.2) (layer "F.Cu") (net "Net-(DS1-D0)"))
 (via (at 119.841765 65.658235) (size 0.6) (drill 0.3) (layers "F.Cu" "B.Cu") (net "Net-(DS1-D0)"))
 (via (at 119.85858 108.64142) (size 0.6) (drill 0.3) (layers "F.Cu" "B.Cu") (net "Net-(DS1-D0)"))
 (via (at 119.01005 109.489949) (size 0.6) (drill 0.3) (layers "F.Cu" "B.Cu") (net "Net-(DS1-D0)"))
 (via (at 117.913753 105.954873) (size 0.6) (drill 0.3) (layers "F.Cu" "B.Cu") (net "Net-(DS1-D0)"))
 (segment (start 121 113.5) (end 121 112.5) (width 0.2) (layer "B.Cu") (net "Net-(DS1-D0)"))
 (segment (start 119.015 104.853626) (end 119.015 58.06) (width 0.2) (layer "B.Cu") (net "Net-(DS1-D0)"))
 (segment (start 119.01005 109.489949) (end 119.01005 110.358579) (width 0.2) (layer "B.Cu") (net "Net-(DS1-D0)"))
 (segment (start 121 112.348529) (end 121 113.5) (width 0.2) (layer "B.Cu") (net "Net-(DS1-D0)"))
 (segment (start 119.85858 65.67505) (end 119.85858 108.64142) (width 0.2) (layer "B.Cu") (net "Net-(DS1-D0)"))
 (segment (start 117.913753 105.954873) (end 119.015 104.853626) (width 0.2) (layer "B.Cu") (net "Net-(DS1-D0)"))
 (segment (start 119.01005 110.358579) (end 121 112.348529) (width 0.2) (layer "B.Cu") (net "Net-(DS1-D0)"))
 (segment (start 119.841765 65.658235) (end 119.85858 65.67505) (width 0.2) (layer "B.Cu") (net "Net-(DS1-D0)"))
 (segment (start 121.575 113.075) (end 121.575 112.075) (width 0.2) (layer "F.Cu") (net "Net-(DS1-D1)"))
 (segment (start 121 111.5) (end 121 109.04112) (width 0.2) (layer "F.Cu") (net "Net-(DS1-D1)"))
 (segment (start 121.575 112.075) (end 121 111.5) (width 0.2) (layer "F.Cu") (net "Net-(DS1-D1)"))
 (segment (start 121.555 58.06) (end 127.5 64.005) (width 0.2) (layer "F.Cu") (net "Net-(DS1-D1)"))
 (segment (start 127.5 64.005) (end 127.5 111.5) (width 0.2) (layer "F.Cu") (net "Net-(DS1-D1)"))
 (segment (start 121 109.04112) (end 120.97944 109.02056) (width 0.2) (layer "F.Cu") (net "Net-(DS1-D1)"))
 (via (at 120.97944 109.02056) (size 0.6) (drill 0.3) (layers "F.Cu" "B.Cu") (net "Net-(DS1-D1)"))
 (segment (start 121.555 108.445) (end 121.555 58.06) (width 0.2) (layer "B.Cu") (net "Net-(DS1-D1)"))
 (segment (start 120.97944 109.02056) (end 121.555 108.445) (width 0.2) (layer "B.Cu") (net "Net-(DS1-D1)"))
 (segment (start 124.095 58.06) (end 128.30444 62.26944) (width 0.2) (layer "F.Cu") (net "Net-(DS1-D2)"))
 (segment (start 122.5 115) (end 126.4 115) (width 0.2) (layer "F.Cu") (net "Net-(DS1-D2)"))
 (segment (start 128.30444 62.26944) (end 128.30444 112.80444) (width 0.2) (layer "F.Cu") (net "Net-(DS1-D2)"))
 (segment (start 122.575 113.075) (end 122.575 114.925) (width 0.2) (layer "F.Cu") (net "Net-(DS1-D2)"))
 (segment (start 122.575 114.925) (end 122.5 115) (width 0.2) (layer "F.Cu") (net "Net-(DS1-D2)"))
 (segment (start 126.4 115) (end 126.5 114.9) (width 0.2) (layer "F.Cu") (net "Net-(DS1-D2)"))
 (via (at 126.5 114.9) (size 0.6) (drill 0.3) (layers "F.Cu" "B.Cu") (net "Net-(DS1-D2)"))
 (via (at 128.30444 112.80444) (size 0.6) (drill 0.3) (layers "F.Cu" "B.Cu") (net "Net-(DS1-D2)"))
 (segment (start 128.30444 113.09556) (end 126.5 114.9) (width 0.2) (layer "B.Cu") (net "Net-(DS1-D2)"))
 (segment (start 128.30444 112.80444) (end 128.30444 113.09556) (width 0.2) (layer "B.Cu") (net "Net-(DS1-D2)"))
 (segment (start 129.825735 105.825735) (end 128.70444 106.947032) (width 0.2) (layer "F.Cu") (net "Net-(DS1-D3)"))
 (segment (start 124.7 110.951473) (end 124.607412 110.951473) (width 0.2) (layer "F.Cu") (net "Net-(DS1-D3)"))
 (segment (start 129.174265 106.477207) (end 128.90444 106.747032) (width 0.2) (layer "F.Cu") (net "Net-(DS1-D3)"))
 (segment (start 126.635 58.06) (end 129.174265 60.599265) (width 0.2) (layer "F.Cu") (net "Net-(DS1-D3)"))
 (segment (start 124.607412 110.951473) (end 123.32797 109.672031) (width 0.2) (layer "F.Cu") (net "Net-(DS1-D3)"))
 (segment (start 129.174265 60.599265) (end 129.174265 106.477207) (width 0.2) (layer "F.Cu") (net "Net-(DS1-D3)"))
 (via (at 124.7 110.951473) (size 0.6) (drill 0.3) (layers "F.Cu" "B.Cu") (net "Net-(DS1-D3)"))
 (via (at 128.90444 106.747032) (size 0.6) (drill 0.3) (layers "F.Cu" "B.Cu") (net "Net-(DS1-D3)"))
 (via (at 123.32797 109.672031) (size 0.6) (drill 0.3) (layers "F.Cu" "B.Cu") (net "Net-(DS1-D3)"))
 (via (at 129.825735 105.825735) (size 0.6) (drill 0.3) (layers "F.Cu" "B.Cu") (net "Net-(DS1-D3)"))
 (segment (start 128.90444 106.747033) (end 124.7 110.951473) (width 0.2) (layer "B.Cu") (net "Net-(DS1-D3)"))
 (segment (start 128.677944 56.46) (end 132.212056 56.46) (width 0.2) (layer "B.Cu") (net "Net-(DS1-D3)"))
 (segment (start 132.915 101.585) (end 129.825735 104.674265) (width 0.2) (layer "B.Cu") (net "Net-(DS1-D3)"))
 (segment (start 129.825735 104.674265) (end 129.825735 105.825735) (width 0.2) (layer "B.Cu") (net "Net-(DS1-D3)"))
 (segment (start 122.5 110.500001) (end 122.5 112.934314) (width 0.2) (layer "B.Cu") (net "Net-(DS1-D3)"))
 (segment (start 132.212056 56.46) (end 132.915 57.162944) (width 0.2) (layer "B.Cu") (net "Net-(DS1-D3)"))
 (segment (start 123.032843 62.105101) (end 127.137944 58) (width 0.2) (layer "B.Cu") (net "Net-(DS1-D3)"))
 (segment (start 123 62.137944) (end 128.677944 56.46) (width 0.2) (layer "B.Cu") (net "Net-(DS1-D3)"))
 (segment (start 123.032843 113.467157) (end 123.032843 62.105101) (width 0.2) (layer "B.Cu") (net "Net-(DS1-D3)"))
 (segment (start 132.915 57.162944) (end 132.915 101.585) (width 0.2) (layer "B.Cu") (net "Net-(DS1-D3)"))
 (segment (start 123 113) (end 123 62.137944) (width 0.2) (layer "B.Cu") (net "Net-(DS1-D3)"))
 (segment (start 123.32797 109.672031) (end 122.5 110.500001) (width 0.2) (layer "B.Cu") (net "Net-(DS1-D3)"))
 (segment (start 122.5 112.934314) (end 123.032843 113.467157) (width 0.2) (layer "B.Cu") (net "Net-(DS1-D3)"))
 (segment (start 125.5 112) (end 123.84259 112) (width 0.2) (layer "F.Cu") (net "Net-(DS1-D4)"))
 (segment (start 123.84259 112) (end 123.575 112.26759) (width 0.2) (layer "F.Cu") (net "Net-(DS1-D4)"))
 (segment (start 123.575 112.26759) (end 123.575 113.075) (width 0.2) (layer "F.Cu") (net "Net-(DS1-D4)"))
 (segment (start 130.5 59.385) (end 130.5 72) (width 0.2) (layer "F.Cu") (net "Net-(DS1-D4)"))
 (segment (start 125.5 112) (end 125.5 109.42078) (width 0.2) (layer "F.Cu") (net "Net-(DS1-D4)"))
 (segment (start 130.5 72) (end 130 72.5) (width 0.2) (layer "F.Cu") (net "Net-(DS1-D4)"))
 (segment (start 129.175 58.06) (end 130.5 59.385) (width 0.2) (layer "F.Cu") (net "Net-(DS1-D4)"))
 (segment (start 125.5 109.42078) (end 124.7 108.62078) (width 0.2) (layer "F.Cu") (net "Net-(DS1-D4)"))
 (via (at 125.5 107.5) (size 0.6) (drill 0.3) (layers "F.Cu" "B.Cu") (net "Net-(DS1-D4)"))
 (via (at 124.7 108.62078) (size 0.6) (drill 0.3) (layers "F.Cu" "B.Cu") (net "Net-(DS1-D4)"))
 (via (at 130 72.5) (size 0.6) (drill 0.3) (layers "F.Cu" "B.Cu") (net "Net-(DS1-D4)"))
 (via (at 125.5 107.5) (size 0.6) (drill 0.3) (layers "F.Cu" "B.Cu") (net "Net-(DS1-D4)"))
 (segment (start 124.734314 108.9) (end 124.7 108.865686) (width 0.2) (layer "B.Cu") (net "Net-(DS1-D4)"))
 (segment (start 129.175 58.06) (end 129.533423 58.06) (width 0.2) (layer "B.Cu") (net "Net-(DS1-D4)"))
 (segment (start 130 72.5) (end 125.5 77) (width 0.2) (layer "B.Cu") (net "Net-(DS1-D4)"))
 (segment (start 125.5 108.134314) (end 124.734314 108.9) (width 0.2) (layer "B.Cu") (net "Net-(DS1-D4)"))
 (segment (start 125.5 77) (end 125.5 107.5) (width 0.2) (layer "B.Cu") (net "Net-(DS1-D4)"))
 (segment (start 125.5 107.5) (end 125.5 108.134314) (width 0.2) (layer "B.Cu") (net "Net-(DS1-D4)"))
 (segment (start 124.7 108.865686) (end 124.7 108.62078) (width 0.2) (layer "B.Cu") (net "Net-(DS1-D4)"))
 (segment (start 124.217158 113.282842) (end 124.1 113.165685) (width 0.2) (layer "B.Cu") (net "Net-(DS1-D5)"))
 (segment (start 124.1 113.165685) (end 124.1 65.675) (width 0.2) (layer "B.Cu") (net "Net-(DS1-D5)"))
 (segment (start 124.1 65.675) (end 131.715 58.06) (width 0.2) (layer "B.Cu") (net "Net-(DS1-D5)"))
 (segment (start 124.575 112.55) (end 124.575 113.075) (width 0.2) (layer "F.Cu") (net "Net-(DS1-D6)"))
 (segment (start 124.525 112.5) (end 124.575 112.55) (width 0.2) (layer "F.Cu") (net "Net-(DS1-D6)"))
 (segment (start 134.255 58.06) (end 133.56 58.06) (width 0.2) (layer "B.Cu") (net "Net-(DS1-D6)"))
 (segment (start 124.5 112) (end 124.5 112.5) (width 0.2) (layer "B.Cu") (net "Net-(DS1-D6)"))
 (segment (start 133.315 57.5) (end 133.315 57.815) (width 0.2) (layer "B.Cu") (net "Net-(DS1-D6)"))
 (segment (start 133.56 58.06) (end 133.315 57.815) (width 0.2) (layer "B.Cu") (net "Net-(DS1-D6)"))
 (segment (start 134.255 102.245) (end 124.5 112) (width 0.2) (layer "B.Cu") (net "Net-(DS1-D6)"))
 (segment (start 134.255 58.06) (end 134.255 102.245) (width 0.2) (layer "B.Cu") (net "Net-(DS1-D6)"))
 (segment (start 136.795 101.205) (end 125.5 112.5) (width 0.2) (layer "B.Cu") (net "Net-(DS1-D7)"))
 (segment (start 125.5 112.5) (end 125.5 113.5) (width 0.2) (layer "B.Cu") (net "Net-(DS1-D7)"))
 (segment (start 136.795 58.06) (end 136.795 101.205) (width 0.2) (layer "B.Cu") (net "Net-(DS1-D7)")))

